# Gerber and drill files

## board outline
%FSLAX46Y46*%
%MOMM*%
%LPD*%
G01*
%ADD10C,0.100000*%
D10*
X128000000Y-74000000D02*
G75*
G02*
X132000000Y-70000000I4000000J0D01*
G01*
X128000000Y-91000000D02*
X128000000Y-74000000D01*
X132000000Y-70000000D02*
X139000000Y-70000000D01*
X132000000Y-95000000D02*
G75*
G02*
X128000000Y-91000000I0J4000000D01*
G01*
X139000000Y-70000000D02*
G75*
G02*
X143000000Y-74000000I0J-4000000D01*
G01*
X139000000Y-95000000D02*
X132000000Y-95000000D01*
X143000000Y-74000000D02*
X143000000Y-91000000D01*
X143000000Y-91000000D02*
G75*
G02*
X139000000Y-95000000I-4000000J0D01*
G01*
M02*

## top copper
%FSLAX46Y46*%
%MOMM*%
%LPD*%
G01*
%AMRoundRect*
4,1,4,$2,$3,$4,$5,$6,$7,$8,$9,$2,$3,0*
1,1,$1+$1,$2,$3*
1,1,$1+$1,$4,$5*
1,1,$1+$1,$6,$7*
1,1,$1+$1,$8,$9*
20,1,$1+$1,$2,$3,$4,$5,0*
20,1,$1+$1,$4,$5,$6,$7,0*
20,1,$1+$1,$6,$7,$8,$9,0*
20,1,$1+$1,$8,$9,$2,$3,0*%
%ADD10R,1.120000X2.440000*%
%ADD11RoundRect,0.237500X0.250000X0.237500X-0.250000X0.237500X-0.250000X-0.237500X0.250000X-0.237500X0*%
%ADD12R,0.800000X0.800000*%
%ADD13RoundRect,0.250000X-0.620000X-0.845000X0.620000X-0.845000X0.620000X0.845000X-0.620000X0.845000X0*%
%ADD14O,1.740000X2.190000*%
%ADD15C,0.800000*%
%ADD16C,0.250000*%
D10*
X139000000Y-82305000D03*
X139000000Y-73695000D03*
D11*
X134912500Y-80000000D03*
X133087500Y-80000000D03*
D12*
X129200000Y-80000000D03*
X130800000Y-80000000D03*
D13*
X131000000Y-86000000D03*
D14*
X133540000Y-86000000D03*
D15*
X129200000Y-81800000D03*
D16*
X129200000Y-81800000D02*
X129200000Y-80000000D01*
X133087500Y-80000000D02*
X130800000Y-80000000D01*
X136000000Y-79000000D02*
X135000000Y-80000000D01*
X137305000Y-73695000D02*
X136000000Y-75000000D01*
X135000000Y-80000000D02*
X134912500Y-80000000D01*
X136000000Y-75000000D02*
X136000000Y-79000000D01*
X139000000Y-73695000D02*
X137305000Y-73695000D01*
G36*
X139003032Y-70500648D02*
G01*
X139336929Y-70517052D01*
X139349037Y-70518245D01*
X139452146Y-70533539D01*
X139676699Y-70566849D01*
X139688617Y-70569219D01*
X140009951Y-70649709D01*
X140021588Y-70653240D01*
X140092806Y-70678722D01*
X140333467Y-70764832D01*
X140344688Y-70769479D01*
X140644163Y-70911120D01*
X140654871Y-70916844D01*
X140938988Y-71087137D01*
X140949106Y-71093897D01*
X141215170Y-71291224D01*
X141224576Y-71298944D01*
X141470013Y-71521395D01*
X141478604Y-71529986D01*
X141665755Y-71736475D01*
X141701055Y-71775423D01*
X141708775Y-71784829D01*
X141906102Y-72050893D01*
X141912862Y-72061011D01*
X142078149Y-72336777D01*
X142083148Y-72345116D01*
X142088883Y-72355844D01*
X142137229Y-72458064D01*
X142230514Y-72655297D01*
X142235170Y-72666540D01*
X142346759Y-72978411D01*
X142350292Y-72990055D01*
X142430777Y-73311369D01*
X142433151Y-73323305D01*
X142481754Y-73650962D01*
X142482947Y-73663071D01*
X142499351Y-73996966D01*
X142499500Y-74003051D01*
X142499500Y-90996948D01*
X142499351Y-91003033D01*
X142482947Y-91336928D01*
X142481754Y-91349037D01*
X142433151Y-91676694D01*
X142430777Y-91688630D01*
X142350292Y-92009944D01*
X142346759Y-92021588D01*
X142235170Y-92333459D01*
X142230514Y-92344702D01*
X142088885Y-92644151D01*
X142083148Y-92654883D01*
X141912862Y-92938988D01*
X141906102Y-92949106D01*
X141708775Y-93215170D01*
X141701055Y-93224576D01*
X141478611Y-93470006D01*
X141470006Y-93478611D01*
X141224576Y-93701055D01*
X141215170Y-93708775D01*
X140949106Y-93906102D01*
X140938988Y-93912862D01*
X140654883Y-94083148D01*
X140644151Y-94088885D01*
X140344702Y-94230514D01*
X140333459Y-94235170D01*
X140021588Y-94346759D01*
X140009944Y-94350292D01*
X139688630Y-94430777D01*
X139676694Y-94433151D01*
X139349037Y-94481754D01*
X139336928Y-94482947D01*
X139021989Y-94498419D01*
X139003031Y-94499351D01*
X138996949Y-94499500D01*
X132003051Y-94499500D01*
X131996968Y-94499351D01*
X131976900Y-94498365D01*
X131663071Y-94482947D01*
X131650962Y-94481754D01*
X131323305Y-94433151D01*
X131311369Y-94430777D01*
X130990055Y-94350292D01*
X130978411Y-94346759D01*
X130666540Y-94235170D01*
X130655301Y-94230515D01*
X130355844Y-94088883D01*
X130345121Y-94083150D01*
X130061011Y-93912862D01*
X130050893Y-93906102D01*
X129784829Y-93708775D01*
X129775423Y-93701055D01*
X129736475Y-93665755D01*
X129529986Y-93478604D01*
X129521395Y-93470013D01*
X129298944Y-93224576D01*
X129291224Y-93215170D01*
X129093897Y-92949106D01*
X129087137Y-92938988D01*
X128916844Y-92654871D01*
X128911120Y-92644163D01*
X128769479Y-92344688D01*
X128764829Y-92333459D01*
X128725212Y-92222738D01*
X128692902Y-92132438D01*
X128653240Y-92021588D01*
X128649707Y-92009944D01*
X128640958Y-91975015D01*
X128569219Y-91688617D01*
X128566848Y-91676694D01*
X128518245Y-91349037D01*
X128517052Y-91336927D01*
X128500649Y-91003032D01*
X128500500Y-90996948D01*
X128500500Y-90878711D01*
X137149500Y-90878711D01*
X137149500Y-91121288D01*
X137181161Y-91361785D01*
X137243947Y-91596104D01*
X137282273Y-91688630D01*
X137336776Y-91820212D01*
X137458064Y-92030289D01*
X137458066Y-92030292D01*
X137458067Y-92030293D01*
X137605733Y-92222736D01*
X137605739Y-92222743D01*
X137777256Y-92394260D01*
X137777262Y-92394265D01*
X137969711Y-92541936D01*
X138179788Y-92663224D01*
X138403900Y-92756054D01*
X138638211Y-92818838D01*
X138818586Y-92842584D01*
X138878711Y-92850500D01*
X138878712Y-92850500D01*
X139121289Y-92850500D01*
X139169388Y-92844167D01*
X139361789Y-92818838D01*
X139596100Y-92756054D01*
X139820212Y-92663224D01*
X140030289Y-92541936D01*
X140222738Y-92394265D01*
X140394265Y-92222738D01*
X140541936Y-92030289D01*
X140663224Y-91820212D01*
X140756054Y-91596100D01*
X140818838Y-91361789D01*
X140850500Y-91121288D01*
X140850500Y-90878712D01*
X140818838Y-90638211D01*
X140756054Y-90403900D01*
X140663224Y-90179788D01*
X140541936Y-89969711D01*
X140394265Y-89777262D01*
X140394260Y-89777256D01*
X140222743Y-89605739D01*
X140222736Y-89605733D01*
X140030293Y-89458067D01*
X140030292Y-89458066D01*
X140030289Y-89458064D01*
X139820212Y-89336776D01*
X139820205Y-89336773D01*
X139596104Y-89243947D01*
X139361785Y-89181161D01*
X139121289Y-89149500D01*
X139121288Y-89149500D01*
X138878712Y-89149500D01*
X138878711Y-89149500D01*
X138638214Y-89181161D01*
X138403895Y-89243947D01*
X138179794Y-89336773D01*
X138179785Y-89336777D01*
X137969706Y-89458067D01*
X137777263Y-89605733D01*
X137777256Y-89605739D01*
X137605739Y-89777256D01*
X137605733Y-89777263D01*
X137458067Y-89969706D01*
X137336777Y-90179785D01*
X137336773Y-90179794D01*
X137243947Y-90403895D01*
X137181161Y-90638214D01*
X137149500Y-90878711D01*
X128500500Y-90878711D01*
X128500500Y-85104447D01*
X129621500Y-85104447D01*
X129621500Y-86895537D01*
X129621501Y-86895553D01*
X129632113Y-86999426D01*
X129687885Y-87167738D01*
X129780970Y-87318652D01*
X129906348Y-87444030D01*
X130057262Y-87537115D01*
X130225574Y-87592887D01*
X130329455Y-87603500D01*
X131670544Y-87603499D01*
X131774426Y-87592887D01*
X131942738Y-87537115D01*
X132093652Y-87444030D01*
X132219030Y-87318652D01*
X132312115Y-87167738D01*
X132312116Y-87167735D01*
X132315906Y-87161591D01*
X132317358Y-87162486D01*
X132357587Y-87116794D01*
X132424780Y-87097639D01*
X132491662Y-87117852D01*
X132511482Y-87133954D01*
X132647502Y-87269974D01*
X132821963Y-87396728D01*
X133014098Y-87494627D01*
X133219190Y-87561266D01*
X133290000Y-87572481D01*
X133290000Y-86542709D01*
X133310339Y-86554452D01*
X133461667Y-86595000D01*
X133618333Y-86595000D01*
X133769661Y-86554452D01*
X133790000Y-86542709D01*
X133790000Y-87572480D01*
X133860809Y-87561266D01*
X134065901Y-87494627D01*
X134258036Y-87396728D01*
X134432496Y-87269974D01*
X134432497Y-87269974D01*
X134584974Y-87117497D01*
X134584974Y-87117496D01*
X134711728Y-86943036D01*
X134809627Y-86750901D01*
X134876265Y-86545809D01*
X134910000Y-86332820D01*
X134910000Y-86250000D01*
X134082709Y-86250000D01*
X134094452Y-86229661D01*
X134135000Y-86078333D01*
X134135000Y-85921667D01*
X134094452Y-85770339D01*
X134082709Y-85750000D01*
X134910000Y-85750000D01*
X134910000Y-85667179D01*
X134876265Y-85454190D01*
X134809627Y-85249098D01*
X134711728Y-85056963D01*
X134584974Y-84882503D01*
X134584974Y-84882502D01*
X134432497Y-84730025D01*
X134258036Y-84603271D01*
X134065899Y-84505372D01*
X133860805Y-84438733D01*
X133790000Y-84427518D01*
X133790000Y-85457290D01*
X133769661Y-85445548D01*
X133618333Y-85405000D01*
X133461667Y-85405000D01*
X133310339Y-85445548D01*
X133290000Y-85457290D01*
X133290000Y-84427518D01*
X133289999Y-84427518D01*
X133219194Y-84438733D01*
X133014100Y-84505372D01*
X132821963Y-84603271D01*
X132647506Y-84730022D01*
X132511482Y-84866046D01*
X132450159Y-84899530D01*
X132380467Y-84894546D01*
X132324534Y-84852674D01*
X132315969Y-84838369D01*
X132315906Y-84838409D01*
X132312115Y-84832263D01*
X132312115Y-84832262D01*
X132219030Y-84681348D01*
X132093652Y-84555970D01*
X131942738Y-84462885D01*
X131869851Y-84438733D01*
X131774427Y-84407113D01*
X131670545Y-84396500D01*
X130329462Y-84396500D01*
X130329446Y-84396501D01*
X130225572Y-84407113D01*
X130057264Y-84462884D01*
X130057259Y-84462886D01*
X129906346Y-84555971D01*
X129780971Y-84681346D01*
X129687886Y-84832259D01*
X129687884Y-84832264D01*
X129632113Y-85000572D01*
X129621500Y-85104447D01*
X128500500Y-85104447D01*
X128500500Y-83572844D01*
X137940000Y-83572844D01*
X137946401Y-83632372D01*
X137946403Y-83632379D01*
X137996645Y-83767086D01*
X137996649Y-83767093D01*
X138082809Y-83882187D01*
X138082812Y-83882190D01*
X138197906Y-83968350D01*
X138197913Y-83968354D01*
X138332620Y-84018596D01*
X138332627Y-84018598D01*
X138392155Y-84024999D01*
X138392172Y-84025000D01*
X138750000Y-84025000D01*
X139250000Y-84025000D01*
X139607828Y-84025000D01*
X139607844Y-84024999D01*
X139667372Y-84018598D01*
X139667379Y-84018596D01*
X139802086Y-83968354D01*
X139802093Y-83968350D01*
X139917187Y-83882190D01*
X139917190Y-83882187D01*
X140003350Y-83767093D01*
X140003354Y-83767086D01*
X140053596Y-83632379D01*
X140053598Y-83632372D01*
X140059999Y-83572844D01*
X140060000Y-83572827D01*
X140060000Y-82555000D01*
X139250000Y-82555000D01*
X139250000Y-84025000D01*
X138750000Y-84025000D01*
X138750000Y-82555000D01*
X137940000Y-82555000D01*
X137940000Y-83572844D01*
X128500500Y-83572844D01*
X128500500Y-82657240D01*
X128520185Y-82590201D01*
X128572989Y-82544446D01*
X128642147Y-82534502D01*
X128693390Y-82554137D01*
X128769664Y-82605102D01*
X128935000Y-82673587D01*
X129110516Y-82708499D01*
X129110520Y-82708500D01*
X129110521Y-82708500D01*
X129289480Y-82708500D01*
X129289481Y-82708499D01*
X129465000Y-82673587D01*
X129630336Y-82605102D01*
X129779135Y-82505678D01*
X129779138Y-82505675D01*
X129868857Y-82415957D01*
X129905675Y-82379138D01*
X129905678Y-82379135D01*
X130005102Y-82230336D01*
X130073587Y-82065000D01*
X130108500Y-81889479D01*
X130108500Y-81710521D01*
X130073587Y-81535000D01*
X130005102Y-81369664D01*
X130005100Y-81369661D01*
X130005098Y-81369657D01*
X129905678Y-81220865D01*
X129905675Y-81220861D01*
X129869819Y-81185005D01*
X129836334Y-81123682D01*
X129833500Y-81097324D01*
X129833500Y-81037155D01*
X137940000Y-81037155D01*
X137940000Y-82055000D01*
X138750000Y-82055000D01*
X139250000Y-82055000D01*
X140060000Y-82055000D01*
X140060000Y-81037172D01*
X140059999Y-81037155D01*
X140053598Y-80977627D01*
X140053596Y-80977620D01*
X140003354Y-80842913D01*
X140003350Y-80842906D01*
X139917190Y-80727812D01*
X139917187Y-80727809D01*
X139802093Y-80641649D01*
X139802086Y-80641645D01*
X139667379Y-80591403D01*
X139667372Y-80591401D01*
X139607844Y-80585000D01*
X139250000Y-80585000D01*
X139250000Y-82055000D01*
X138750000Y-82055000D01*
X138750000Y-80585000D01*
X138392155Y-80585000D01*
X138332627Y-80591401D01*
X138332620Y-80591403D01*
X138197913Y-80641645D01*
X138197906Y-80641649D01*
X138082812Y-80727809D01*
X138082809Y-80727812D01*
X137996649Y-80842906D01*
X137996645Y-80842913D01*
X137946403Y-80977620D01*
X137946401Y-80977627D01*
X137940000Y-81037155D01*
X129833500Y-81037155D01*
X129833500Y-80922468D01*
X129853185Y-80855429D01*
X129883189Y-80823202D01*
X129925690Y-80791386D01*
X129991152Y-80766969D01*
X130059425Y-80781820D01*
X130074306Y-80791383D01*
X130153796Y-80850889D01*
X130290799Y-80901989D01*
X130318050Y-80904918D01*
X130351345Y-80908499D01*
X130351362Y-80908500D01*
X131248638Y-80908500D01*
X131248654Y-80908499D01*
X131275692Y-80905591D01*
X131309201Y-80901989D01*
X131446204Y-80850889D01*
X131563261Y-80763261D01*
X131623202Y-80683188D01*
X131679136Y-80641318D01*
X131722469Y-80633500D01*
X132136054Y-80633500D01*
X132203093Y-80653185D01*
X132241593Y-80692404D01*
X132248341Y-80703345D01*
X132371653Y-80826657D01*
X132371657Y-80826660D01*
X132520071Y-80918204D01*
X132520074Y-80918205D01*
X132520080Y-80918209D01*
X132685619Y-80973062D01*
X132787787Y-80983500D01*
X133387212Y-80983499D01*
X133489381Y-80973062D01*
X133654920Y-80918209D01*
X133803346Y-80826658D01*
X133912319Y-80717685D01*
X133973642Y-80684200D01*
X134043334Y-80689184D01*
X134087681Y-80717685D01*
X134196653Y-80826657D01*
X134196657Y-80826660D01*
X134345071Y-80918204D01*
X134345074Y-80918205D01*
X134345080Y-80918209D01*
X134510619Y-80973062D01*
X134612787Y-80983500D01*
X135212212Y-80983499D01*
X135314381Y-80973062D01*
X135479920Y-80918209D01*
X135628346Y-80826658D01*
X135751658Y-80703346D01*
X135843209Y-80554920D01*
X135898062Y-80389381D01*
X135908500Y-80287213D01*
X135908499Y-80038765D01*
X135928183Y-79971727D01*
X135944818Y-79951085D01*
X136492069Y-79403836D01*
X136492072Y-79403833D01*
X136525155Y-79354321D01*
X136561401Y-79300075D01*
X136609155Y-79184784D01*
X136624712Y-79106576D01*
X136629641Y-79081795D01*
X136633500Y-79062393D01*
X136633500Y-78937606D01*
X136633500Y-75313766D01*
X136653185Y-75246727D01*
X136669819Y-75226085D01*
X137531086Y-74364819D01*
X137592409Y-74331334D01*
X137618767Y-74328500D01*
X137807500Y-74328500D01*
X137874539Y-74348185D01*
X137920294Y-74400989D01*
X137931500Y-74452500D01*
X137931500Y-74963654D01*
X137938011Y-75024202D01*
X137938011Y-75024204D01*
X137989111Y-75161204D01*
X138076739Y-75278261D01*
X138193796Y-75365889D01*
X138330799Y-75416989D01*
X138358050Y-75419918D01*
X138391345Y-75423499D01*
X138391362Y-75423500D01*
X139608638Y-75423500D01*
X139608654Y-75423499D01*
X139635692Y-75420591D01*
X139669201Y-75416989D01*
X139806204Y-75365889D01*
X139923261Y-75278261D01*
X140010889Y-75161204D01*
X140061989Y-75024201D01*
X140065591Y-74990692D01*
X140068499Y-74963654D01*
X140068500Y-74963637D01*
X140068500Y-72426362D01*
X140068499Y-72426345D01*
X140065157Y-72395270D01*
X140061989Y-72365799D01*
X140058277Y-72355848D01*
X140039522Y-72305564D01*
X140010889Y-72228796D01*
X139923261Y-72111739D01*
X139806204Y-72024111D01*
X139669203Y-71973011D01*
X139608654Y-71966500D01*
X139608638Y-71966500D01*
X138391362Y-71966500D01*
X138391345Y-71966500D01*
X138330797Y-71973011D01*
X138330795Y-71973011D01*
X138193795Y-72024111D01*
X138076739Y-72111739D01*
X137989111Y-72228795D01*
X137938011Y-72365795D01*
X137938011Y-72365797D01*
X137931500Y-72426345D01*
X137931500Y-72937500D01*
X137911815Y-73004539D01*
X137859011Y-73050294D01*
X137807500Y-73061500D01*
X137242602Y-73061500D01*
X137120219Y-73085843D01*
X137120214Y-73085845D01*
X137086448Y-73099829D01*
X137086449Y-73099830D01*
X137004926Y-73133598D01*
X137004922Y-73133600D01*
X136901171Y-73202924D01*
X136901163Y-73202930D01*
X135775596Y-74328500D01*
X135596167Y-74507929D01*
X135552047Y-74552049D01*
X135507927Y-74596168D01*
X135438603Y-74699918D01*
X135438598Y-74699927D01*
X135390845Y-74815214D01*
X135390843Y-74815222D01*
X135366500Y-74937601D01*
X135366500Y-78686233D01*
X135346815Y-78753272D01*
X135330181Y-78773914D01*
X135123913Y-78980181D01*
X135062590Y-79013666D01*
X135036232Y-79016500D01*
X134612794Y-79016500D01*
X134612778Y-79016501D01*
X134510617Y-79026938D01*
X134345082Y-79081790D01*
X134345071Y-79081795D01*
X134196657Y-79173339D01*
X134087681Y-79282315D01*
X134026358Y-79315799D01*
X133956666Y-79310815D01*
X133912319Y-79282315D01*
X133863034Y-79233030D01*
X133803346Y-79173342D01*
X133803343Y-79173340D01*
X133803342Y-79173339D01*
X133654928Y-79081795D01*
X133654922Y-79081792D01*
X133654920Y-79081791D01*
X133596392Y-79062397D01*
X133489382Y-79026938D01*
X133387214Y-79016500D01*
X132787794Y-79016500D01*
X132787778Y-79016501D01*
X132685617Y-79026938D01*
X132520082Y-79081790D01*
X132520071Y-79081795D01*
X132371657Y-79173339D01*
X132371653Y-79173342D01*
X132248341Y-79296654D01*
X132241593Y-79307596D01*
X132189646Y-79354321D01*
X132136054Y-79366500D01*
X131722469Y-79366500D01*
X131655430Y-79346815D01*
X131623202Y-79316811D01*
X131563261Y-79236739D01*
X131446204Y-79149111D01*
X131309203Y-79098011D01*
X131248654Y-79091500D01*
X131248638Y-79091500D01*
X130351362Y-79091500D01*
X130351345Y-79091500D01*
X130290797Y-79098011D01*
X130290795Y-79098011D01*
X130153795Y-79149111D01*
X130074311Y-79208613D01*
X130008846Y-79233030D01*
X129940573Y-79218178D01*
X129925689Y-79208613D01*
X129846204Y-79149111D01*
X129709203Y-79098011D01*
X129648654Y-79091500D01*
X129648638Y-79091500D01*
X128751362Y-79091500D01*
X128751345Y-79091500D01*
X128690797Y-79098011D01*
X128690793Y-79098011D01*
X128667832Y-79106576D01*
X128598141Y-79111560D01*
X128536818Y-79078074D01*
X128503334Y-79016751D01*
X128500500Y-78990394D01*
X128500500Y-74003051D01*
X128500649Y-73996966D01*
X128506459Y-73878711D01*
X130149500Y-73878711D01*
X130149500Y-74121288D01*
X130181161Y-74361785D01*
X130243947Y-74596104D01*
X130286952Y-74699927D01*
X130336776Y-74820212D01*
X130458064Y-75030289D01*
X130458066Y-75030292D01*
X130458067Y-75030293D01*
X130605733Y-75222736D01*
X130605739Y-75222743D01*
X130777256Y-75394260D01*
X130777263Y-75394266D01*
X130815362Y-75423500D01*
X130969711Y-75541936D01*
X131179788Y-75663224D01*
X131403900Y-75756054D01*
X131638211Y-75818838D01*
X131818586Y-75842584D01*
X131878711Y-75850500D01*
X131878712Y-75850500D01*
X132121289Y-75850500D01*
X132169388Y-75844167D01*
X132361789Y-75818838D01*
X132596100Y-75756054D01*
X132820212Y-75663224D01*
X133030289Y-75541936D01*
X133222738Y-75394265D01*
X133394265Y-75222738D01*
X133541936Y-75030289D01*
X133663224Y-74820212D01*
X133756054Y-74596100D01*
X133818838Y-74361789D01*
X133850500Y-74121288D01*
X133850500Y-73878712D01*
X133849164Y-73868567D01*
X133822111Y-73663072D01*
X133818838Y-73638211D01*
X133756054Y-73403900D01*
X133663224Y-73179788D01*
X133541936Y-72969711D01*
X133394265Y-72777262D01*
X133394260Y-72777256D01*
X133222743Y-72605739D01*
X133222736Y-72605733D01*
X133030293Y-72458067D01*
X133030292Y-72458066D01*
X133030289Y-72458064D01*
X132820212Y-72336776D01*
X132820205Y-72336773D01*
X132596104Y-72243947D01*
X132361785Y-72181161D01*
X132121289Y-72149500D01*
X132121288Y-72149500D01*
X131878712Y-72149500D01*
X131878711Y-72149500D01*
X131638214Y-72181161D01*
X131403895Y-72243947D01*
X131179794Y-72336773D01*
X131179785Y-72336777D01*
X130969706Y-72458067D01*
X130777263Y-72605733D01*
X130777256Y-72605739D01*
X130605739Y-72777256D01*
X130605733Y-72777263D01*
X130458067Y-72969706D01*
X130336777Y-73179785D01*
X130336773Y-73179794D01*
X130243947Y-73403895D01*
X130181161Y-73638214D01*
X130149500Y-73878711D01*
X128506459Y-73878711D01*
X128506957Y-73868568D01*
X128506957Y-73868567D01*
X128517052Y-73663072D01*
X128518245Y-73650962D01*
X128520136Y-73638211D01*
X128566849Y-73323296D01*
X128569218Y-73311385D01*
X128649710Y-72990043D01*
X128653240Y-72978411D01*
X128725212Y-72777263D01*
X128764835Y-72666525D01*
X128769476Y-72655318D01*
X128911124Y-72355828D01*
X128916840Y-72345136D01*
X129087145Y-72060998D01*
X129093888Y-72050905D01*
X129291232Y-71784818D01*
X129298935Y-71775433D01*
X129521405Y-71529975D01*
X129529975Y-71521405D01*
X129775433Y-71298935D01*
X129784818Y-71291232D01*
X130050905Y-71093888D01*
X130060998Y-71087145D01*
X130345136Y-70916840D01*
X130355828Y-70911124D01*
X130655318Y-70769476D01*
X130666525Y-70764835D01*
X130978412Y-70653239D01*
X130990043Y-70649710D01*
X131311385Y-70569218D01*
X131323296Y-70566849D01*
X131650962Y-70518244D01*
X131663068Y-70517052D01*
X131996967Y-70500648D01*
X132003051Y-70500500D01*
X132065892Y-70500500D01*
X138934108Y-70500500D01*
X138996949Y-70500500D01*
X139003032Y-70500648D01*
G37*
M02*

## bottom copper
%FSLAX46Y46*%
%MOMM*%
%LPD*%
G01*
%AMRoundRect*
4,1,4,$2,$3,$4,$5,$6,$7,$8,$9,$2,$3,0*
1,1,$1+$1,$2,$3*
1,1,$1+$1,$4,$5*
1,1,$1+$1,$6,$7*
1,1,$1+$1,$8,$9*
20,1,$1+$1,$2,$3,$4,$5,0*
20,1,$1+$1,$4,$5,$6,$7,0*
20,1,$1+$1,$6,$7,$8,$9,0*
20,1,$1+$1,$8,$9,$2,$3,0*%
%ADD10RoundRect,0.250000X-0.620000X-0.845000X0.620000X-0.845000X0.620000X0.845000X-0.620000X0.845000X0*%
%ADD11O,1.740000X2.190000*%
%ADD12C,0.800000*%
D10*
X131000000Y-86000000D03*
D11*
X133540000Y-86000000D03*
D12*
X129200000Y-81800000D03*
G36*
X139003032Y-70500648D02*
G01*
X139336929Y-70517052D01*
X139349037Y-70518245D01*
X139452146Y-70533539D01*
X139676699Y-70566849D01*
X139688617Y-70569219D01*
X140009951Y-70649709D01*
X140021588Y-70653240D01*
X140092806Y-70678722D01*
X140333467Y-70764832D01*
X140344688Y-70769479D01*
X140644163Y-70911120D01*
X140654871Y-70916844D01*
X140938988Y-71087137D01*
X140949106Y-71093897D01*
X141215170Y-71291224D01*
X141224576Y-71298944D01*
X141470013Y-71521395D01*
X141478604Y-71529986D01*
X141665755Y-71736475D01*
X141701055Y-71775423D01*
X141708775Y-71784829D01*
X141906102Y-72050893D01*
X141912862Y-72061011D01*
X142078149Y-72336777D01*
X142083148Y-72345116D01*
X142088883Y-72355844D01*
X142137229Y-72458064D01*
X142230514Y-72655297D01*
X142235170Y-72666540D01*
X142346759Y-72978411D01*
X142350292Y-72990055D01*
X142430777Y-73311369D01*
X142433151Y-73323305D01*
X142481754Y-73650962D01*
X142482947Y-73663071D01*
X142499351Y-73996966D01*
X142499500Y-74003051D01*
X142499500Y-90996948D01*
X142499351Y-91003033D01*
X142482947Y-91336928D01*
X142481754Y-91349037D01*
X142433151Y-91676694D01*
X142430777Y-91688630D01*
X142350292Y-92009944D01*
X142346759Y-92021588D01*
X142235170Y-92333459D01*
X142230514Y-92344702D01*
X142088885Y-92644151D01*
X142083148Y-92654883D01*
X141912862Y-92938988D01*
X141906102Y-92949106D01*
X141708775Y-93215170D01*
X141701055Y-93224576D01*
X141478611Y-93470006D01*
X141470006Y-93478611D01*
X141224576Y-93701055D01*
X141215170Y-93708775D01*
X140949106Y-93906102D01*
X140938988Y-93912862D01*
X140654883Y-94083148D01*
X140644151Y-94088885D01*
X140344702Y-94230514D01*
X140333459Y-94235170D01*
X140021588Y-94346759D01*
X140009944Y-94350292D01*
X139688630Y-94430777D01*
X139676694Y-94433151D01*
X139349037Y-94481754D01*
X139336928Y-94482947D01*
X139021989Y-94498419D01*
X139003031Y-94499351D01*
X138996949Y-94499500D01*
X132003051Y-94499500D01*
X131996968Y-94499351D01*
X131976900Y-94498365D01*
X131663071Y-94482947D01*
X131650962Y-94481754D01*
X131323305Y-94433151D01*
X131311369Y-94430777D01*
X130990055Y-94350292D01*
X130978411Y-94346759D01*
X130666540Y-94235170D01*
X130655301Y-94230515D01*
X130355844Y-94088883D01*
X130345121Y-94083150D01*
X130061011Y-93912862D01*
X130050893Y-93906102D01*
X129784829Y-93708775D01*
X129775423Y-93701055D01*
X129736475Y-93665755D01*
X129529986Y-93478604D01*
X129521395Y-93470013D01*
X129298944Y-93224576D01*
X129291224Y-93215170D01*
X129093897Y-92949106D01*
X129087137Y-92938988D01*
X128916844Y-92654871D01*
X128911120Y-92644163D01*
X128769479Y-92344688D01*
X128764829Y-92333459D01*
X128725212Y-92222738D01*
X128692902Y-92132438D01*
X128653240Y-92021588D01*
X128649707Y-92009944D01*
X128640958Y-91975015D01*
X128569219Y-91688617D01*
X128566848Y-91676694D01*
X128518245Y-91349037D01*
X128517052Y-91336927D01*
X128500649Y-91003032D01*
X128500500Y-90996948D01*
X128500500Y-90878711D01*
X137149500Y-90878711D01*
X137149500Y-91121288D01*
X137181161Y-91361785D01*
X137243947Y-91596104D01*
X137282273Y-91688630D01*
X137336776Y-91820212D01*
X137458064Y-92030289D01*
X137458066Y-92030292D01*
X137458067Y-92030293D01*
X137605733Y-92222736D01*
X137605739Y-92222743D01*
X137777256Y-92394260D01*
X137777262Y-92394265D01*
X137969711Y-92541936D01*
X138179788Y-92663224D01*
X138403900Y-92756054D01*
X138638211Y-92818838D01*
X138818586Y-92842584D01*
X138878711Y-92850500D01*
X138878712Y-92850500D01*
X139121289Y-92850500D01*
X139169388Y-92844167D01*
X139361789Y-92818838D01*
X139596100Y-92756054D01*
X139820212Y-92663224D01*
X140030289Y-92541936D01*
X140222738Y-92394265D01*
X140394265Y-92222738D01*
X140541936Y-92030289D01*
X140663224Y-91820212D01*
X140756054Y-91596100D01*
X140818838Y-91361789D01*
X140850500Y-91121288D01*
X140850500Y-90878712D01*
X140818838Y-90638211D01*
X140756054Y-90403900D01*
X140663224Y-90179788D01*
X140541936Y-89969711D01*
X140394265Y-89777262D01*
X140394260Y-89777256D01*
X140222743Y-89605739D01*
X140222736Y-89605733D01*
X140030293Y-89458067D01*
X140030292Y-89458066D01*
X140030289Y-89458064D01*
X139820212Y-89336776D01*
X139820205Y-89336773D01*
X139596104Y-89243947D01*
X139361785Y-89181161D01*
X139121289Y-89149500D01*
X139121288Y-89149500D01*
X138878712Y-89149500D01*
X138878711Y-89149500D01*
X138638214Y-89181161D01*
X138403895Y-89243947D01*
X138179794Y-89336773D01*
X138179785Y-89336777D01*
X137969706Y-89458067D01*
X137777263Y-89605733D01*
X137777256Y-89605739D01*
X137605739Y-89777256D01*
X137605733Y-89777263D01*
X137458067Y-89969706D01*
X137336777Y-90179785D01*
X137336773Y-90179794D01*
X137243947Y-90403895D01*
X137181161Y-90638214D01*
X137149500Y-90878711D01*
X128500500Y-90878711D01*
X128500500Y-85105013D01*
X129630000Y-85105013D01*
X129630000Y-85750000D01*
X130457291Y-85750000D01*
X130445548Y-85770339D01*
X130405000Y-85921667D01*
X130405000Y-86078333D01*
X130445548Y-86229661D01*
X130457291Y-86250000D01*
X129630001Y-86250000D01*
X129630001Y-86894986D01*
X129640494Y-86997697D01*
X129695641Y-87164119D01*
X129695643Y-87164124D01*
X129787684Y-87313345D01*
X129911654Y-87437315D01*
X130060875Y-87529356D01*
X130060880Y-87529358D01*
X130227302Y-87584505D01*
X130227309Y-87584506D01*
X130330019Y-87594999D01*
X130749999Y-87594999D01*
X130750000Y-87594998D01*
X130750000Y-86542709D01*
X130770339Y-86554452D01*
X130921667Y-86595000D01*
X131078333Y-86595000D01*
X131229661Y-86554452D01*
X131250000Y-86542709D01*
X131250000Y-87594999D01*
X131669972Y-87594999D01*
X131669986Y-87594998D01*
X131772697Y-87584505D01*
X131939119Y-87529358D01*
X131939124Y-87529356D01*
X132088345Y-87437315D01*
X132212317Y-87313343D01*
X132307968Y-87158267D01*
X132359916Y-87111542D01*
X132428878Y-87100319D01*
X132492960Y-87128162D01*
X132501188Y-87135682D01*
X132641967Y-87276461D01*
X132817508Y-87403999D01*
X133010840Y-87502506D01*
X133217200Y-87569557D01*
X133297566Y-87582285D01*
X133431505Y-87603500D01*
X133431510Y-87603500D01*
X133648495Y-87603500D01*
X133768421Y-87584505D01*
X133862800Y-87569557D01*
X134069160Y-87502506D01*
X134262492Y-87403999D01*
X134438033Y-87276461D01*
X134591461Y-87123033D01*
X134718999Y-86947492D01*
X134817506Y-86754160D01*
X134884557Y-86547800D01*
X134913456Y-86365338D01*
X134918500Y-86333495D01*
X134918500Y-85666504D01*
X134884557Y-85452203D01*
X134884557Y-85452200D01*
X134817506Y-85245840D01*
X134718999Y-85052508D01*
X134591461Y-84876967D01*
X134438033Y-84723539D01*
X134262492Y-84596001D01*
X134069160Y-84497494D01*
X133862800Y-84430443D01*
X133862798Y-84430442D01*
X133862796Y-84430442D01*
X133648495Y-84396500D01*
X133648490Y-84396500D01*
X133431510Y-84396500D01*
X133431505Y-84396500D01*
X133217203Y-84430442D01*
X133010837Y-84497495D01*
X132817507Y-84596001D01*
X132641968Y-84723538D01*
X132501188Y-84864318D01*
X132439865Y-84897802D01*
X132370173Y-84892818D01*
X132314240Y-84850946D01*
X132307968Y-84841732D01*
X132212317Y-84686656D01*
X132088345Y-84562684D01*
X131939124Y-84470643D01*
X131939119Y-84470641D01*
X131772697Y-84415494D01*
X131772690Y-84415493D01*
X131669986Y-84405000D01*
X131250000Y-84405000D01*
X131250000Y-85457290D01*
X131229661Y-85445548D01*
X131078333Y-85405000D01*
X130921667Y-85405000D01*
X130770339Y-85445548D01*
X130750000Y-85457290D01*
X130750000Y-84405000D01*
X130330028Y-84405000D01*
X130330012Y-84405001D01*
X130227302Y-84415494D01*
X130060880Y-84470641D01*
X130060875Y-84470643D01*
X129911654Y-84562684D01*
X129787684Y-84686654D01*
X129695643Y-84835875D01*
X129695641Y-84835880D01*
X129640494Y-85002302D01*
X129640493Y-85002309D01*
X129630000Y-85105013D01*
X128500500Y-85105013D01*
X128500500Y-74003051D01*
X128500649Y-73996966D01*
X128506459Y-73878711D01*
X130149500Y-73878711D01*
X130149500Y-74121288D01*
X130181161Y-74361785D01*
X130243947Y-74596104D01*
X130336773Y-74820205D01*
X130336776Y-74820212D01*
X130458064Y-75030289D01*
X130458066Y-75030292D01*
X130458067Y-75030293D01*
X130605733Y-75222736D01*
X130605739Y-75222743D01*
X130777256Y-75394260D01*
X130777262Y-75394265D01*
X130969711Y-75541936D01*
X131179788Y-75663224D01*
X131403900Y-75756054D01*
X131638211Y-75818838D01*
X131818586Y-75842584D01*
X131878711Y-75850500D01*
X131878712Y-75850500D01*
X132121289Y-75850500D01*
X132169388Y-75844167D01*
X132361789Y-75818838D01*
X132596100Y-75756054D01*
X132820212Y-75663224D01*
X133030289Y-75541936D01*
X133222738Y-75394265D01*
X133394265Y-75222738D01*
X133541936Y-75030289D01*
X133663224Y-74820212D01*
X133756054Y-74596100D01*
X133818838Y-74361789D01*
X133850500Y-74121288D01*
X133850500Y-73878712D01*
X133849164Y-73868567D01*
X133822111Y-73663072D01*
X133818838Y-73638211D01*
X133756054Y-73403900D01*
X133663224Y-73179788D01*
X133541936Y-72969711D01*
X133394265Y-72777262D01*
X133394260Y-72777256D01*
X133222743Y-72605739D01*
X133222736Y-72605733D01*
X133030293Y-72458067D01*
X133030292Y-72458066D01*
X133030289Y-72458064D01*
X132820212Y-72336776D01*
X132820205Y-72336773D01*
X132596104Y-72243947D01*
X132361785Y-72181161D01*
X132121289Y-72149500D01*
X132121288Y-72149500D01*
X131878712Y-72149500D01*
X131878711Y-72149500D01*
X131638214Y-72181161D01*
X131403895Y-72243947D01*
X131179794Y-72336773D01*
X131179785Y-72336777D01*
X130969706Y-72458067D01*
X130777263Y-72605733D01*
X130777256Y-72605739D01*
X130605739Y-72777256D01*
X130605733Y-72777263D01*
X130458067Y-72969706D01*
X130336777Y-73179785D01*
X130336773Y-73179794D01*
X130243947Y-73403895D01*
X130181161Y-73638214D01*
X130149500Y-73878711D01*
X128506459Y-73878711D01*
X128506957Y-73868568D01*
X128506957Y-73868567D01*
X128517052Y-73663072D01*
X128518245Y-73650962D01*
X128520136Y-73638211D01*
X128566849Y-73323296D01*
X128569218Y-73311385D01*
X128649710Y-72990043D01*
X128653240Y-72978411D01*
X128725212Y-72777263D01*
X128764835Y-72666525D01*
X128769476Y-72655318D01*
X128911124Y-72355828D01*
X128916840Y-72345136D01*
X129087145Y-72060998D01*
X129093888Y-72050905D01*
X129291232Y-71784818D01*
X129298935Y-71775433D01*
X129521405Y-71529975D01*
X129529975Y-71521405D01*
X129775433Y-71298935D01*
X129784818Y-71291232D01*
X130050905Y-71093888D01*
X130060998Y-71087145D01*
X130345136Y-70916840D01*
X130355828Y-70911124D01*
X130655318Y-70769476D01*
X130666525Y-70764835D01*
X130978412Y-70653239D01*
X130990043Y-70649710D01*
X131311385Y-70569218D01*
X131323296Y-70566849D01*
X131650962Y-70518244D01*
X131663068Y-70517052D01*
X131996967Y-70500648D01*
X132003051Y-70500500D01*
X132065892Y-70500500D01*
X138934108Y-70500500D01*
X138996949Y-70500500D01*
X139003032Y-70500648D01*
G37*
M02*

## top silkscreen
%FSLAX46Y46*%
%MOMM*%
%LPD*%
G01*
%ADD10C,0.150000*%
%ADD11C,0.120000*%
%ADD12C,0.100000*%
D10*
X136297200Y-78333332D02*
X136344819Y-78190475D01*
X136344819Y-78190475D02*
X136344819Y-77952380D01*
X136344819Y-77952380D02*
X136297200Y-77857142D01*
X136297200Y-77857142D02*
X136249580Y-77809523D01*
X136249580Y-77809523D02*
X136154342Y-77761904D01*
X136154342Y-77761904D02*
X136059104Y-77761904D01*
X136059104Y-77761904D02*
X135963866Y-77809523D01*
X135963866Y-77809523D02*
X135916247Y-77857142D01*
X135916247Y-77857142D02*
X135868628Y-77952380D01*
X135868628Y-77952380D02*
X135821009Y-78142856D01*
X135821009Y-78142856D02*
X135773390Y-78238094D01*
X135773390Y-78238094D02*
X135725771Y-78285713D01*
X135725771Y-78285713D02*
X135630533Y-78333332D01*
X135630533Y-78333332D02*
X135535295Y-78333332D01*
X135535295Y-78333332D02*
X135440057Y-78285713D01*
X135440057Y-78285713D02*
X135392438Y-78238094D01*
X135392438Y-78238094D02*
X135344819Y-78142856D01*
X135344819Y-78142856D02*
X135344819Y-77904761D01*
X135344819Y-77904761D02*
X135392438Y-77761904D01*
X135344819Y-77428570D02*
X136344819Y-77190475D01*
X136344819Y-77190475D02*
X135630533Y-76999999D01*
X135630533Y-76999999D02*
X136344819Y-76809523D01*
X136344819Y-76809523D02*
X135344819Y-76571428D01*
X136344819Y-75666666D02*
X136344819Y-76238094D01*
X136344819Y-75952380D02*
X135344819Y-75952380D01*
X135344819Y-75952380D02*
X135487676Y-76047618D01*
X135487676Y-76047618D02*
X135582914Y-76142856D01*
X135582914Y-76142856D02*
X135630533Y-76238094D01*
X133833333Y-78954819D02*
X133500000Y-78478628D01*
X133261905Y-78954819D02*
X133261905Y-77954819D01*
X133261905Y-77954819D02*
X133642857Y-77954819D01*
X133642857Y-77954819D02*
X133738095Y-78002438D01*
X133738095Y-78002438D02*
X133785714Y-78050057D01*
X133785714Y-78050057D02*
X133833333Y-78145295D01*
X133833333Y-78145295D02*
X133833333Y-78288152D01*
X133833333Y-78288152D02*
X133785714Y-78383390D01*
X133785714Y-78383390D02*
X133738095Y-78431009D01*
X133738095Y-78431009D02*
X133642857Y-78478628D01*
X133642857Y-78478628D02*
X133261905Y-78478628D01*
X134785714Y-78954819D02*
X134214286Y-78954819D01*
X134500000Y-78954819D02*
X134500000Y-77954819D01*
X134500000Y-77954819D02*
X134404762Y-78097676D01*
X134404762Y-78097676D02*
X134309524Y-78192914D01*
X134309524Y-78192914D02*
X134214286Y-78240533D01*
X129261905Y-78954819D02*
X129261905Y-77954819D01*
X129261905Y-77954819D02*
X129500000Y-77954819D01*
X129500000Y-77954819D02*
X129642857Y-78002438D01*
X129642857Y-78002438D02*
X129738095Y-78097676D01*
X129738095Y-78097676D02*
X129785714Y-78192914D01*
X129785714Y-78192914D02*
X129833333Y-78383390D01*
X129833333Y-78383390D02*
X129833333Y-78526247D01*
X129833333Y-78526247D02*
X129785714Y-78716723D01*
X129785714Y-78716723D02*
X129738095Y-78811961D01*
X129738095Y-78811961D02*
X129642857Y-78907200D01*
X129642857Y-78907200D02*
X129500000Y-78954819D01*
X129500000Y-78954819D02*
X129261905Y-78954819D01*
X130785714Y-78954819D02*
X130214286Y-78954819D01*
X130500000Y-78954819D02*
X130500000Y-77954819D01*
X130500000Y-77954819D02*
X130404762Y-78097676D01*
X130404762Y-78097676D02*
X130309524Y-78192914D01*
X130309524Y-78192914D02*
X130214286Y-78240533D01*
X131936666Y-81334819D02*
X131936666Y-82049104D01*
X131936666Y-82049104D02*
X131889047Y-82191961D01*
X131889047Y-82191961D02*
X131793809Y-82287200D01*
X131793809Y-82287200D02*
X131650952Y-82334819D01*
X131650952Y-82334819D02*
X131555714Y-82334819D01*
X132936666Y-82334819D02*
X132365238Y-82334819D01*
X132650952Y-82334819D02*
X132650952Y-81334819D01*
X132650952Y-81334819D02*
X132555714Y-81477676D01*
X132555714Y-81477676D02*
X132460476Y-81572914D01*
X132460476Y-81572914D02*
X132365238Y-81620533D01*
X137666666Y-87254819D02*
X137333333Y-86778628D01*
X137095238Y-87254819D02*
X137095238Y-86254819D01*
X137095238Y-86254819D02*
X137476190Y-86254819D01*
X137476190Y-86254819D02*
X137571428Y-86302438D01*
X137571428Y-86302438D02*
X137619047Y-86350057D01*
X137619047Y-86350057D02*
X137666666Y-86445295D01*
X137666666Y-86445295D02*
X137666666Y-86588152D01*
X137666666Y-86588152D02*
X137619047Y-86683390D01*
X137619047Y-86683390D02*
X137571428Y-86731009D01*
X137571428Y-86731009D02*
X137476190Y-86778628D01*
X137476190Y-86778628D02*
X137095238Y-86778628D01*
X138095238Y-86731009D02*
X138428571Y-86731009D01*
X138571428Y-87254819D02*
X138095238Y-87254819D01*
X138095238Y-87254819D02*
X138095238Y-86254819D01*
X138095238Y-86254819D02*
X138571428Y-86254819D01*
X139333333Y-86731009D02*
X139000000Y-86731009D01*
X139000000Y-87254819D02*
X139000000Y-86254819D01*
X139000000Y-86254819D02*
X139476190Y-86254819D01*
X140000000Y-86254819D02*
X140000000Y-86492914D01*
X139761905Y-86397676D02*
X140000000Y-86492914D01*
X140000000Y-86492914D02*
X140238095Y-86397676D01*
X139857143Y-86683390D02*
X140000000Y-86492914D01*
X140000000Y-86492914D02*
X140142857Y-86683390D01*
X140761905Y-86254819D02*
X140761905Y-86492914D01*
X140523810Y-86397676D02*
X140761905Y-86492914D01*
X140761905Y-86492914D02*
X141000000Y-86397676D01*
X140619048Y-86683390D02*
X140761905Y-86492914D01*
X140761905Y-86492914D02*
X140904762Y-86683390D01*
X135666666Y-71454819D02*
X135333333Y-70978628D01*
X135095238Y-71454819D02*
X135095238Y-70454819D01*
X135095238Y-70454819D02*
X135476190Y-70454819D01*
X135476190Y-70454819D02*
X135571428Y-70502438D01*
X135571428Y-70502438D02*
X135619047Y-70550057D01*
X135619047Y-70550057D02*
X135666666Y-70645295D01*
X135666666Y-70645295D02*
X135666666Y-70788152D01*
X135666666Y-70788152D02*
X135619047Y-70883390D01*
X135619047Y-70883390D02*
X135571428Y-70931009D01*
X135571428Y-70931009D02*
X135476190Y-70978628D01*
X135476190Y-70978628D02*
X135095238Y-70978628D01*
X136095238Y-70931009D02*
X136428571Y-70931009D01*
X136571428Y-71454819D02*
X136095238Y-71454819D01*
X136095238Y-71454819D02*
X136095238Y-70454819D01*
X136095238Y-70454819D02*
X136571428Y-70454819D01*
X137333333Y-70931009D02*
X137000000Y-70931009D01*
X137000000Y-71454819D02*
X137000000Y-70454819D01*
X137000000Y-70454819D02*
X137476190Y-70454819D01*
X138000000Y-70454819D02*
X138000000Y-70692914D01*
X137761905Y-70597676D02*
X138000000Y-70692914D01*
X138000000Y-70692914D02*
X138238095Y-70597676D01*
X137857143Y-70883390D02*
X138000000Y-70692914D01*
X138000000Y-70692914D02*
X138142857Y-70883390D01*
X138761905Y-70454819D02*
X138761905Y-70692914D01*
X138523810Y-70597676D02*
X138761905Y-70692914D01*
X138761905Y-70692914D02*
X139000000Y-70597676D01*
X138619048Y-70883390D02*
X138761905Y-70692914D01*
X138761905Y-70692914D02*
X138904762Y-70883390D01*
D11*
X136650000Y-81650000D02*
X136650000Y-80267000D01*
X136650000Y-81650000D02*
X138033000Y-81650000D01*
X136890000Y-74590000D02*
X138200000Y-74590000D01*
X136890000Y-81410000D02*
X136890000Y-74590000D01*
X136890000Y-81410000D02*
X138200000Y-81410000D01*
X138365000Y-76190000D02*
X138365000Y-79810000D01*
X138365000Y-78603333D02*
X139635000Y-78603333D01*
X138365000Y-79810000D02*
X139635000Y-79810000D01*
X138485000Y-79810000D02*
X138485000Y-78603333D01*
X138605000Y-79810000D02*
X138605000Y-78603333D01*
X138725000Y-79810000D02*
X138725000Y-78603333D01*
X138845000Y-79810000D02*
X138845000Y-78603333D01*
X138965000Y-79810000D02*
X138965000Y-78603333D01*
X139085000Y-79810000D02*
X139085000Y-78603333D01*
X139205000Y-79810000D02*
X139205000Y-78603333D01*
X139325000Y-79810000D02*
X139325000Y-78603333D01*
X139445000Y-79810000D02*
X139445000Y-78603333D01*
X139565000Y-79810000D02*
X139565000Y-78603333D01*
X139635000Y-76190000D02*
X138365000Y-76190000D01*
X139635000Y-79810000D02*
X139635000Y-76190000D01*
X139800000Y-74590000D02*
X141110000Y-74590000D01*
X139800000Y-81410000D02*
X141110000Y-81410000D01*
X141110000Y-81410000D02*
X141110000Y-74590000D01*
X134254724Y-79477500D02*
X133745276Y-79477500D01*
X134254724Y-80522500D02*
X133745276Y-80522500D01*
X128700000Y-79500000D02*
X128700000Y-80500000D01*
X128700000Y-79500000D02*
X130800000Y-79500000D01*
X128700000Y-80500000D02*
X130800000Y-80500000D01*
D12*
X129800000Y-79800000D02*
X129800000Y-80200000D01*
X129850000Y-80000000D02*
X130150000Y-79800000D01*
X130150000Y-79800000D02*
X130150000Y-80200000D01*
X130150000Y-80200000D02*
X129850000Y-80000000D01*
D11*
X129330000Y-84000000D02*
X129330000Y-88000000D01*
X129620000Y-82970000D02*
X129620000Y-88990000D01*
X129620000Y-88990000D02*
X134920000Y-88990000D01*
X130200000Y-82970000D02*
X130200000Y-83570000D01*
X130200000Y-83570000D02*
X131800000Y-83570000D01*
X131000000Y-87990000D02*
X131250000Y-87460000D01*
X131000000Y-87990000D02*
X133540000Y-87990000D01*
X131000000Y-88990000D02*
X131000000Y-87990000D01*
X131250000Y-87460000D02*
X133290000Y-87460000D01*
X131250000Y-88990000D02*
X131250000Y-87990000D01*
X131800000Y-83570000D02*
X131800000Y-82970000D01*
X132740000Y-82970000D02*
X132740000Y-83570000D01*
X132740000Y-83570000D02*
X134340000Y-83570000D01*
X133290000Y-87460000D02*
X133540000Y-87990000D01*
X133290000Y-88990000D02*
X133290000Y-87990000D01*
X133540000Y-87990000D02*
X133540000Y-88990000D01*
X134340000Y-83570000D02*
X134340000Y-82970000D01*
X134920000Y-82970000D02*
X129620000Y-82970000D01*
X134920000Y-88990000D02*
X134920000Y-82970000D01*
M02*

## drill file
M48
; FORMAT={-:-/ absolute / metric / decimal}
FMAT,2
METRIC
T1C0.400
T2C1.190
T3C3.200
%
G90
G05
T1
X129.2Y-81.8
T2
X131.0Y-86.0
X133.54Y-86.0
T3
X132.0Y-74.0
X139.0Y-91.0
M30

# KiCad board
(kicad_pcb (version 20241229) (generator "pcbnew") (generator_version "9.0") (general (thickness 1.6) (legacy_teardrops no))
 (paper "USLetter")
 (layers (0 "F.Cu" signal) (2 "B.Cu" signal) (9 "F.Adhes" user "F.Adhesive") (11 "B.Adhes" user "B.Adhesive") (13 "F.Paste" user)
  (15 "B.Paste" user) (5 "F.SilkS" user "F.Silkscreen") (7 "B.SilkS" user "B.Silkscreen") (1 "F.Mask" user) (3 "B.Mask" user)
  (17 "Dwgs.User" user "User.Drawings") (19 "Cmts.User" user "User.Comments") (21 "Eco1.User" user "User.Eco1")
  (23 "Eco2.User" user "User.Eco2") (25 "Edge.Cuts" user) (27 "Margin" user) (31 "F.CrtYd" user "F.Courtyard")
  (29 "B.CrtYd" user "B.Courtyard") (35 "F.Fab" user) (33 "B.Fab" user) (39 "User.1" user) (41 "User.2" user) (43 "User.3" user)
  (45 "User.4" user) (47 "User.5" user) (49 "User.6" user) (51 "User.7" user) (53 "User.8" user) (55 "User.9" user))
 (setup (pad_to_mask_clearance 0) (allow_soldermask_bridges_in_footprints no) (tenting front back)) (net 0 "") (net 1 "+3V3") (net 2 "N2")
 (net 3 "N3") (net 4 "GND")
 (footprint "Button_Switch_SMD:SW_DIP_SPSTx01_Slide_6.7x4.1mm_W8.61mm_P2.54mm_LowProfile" (layer "F.Cu") (at 139 78 90)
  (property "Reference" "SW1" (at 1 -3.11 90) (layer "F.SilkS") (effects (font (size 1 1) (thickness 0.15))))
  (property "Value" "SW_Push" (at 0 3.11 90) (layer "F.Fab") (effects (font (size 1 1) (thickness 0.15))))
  (fp_line (start -3.65 -2.35) (end -2.267 -2.35) (stroke (width 0.12) (type solid)) (layer "F.SilkS"))
  (fp_line (start -3.65 -2.35) (end -3.65 -0.967) (stroke (width 0.12) (type solid)) (layer "F.SilkS"))
  (fp_line (start 3.41 -2.11) (end 3.41 -0.8) (stroke (width 0.12) (type solid)) (layer "F.SilkS"))
  (fp_line (start -3.41 -2.11) (end 3.41 -2.11) (stroke (width 0.12) (type solid)) (layer "F.SilkS"))
  (fp_line (start -3.41 -2.11) (end -3.41 -0.8) (stroke (width 0.12) (type solid)) (layer "F.SilkS"))
  (fp_line (start 1.81 -0.635) (end -1.81 -0.635) (stroke (width 0.12) (type solid)) (layer "F.SilkS"))
  (fp_line (start -0.603333 -0.635) (end -0.603333 0.635) (stroke (width 0.12) (type solid)) (layer "F.SilkS"))
  (fp_line (start -1.81 -0.635) (end -1.81 0.635) (stroke (width 0.12) (type solid)) (layer "F.SilkS"))
  (fp_line (start -1.81 -0.515) (end -0.603333 -0.515) (stroke (width 0.12) (type solid)) (layer "F.SilkS"))
  (fp_line (start -1.81 -0.395) (end -0.603333 -0.395) (stroke (width 0.12) (type solid)) (layer "F.SilkS"))
  (fp_line (start -1.81 -0.275) (end -0.603333 -0.275) (stroke (width 0.12) (type solid)) (layer "F.SilkS"))
  (fp_line (start -1.81 -0.155) (end -0.603333 -0.155) (stroke (width 0.12) (type solid)) (layer "F.SilkS"))
  (fp_line (start -1.81 -0.035) (end -0.603333 -0.035) (stroke (width 0.12) (type solid)) (layer "F.SilkS"))
  (fp_line (start -1.81 0.085) (end -0.603333 0.085) (stroke (width 0.12) (type solid)) (layer "F.SilkS"))
  (fp_line (start -1.81 0.205) (end -0.603333 0.205) (stroke (width 0.12) (type solid)) (layer "F.SilkS"))
  (fp_line (start -1.81 0.325) (end -0.603333 0.325) (stroke (width 0.12) (type solid)) (layer "F.SilkS"))
  (fp_line (start -1.81 0.445) (end -0.603333 0.445) (stroke (width 0.12) (type solid)) (layer "F.SilkS"))
  (fp_line (start -1.81 0.565) (end -0.603333 0.565) (stroke (width 0.12) (type solid)) (layer "F.SilkS"))
  (fp_line (start 1.81 0.635) (end 1.81 -0.635) (stroke (width 0.12) (type solid)) (layer "F.SilkS"))
  (fp_line (start -1.81 0.635) (end 1.81 0.635) (stroke (width 0.12) (type solid)) (layer "F.SilkS"))
  (fp_line (start 3.41 0.8) (end 3.41 2.11) (stroke (width 0.12) (type solid)) (layer "F.SilkS"))
  (fp_line (start -3.41 0.8) (end -3.41 2.11) (stroke (width 0.12) (type solid)) (layer "F.SilkS"))
  (fp_line (start -3.41 2.11) (end 3.41 2.11) (stroke (width 0.12) (type solid)) (layer "F.SilkS"))
  (pad "1" smd rect (at -4.305 0 90) (size 2.44 1.12) (layers "F.Cu" "F.Mask" "F.Paste") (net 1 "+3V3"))
  (pad "2" smd rect (at 4.305 0 90) (size 2.44 1.12) (layers "F.Cu" "F.Mask" "F.Paste") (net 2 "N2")))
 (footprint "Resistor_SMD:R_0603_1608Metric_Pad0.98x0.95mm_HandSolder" (layer "F.Cu") (at 134 80 180)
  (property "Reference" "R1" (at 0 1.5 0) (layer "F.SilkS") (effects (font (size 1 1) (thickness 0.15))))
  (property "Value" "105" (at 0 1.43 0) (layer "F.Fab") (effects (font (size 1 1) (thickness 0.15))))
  (fp_line (start -0.254724 0.5225) (end 0.254724 0.5225) (stroke (width 0.12) (type solid)) (layer "F.SilkS"))
  (fp_line (start -0.254724 -0.5225) (end 0.254724 -0.5225) (stroke (width 0.12) (type solid)) (layer "F.SilkS"))
  (pad "1" smd roundrect (at -0.9125 0 180) (size 0.975 0.95) (layers "F.Cu" "F.Mask" "F.Paste") (roundrect_rratio 0.25) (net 2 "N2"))
  (pad "2" smd roundrect (at 0.9125 0 180) (size 0.975 0.95) (layers "F.Cu" "F.Mask" "F.Paste") (roundrect_rratio 0.25) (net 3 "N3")))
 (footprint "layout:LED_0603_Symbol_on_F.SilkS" (layer "F.Cu") (at 130 80)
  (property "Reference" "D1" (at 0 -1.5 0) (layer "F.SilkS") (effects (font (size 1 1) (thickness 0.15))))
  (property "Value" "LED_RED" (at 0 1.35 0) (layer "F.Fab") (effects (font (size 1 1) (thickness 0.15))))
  (fp_line (start -1.3 -0.5) (end -1.3 0.5) (stroke (width 0.12) (type solid)) (layer "F.SilkS"))
  (fp_line (start -1.3 -0.5) (end 0.8 -0.5) (stroke (width 0.12) (type solid)) (layer "F.SilkS"))
  (fp_line (start -1.3 0.5) (end 0.8 0.5) (stroke (width 0.12) (type solid)) (layer "F.SilkS"))
  (fp_line (start -0.2 -0.2) (end -0.2 0.2) (stroke (width 0.1) (type solid)) (layer "F.SilkS"))
  (fp_line (start -0.15 0) (end 0.15 -0.2) (stroke (width 0.1) (type solid)) (layer "F.SilkS"))
  (fp_line (start 0.15 -0.2) (end 0.15 0.2) (stroke (width 0.1) (type solid)) (layer "F.SilkS"))
  (fp_line (start 0.15 0.2) (end -0.15 0) (stroke (width 0.1) (type solid)) (layer "F.SilkS"))
  (pad "1" smd rect (at -0.8 0 180) (size 0.8 0.8) (layers "F.Cu" "F.Mask" "F.Paste") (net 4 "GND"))
  (pad "2" smd rect (at 0.8 0 180) (size 0.8 0.8) (layers "F.Cu" "F.Mask" "F.Paste") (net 3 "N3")))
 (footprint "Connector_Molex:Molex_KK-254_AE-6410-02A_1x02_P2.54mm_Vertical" (layer "F.Cu") (at 131 86)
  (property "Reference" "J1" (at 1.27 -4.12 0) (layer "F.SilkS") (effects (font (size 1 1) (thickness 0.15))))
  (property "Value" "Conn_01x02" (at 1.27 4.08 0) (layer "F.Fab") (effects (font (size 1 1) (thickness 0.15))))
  (fp_line (start -1.67 -2) (end -1.67 2) (stroke (width 0.12) (type solid)) (layer "F.SilkS"))
  (fp_line (start -1.38 -3.03) (end -1.38 2.99) (stroke (width 0.12) (type solid)) (layer "F.SilkS"))
  (fp_line (start -1.38 2.99) (end 3.92 2.99) (stroke (width 0.12) (type solid)) (layer "F.SilkS"))
  (fp_line (start -0.8 -3.03) (end -0.8 -2.43) (stroke (width 0.12) (type solid)) (layer "F.SilkS"))
  (fp_line (start -0.8 -2.43) (end 0.8 -2.43) (stroke (width 0.12) (type solid)) (layer "F.SilkS"))
  (fp_line (start 0 1.99) (end 0.25 1.46) (stroke (width 0.12) (type solid)) (layer "F.SilkS"))
  (fp_line (start 0 1.99) (end 2.54 1.99) (stroke (width 0.12) (type solid)) (layer "F.SilkS"))
  (fp_line (start 0 2.99) (end 0 1.99) (stroke (width 0.12) (type solid)) (layer "F.SilkS"))
  (fp_line (start 0.25 1.46) (end 2.29 1.46) (stroke (width 0.12) (type solid)) (layer "F.SilkS"))
  (fp_line (start 0.25 2.99) (end 0.25 1.99) (stroke (width 0.12) (type solid)) (layer "F.SilkS"))
  (fp_line (start 0.8 -2.43) (end 0.8 -3.03) (stroke (width 0.12) (type solid)) (layer "F.SilkS"))
  (fp_line (start 1.74 -3.03) (end 1.74 -2.43) (stroke (width 0.12) (type solid)) (layer "F.SilkS"))
  (fp_line (start 1.74 -2.43) (end 3.34 -2.43) (stroke (width 0.12) (type solid)) (layer "F.SilkS"))
  (fp_line (start 2.29 1.46) (end 2.54 1.99) (stroke (width 0.12) (type solid)) (layer "F.SilkS"))
  (fp_line (start 2.29 2.99) (end 2.29 1.99) (stroke (width 0.12) (type solid)) (layer "F.SilkS"))
  (fp_line (start 2.54 1.99) (end 2.54 2.99) (stroke (width 0.12) (type solid)) (layer "F.SilkS"))
  (fp_line (start 3.34 -2.43) (end 3.34 -3.03) (stroke (width 0.12) (type solid)) (layer "F.SilkS"))
  (fp_line (start 3.92 -3.03) (end -1.38 -3.03) (stroke (width 0.12) (type solid)) (layer "F.SilkS"))
  (fp_line (start 3.92 2.99) (end 3.92 -3.03) (stroke (width 0.12) (type solid)) (layer "F.SilkS"))
  (pad "1" thru_hole roundrect (at 0 0) (size 1.74 2.19) (drill 1.19) (layers "*.Cu" "*.Mask") (remove_unused_layers no)
   (roundrect_rratio 0.143678) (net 4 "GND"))
  (pad "2" thru_hole oval (at 2.54 0) (size 1.74 2.19) (drill 1.19) (layers "*.Cu" "*.Mask") (remove_unused_layers no) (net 1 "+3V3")))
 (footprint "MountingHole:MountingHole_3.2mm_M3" (layer "F.Cu") (at 139 91)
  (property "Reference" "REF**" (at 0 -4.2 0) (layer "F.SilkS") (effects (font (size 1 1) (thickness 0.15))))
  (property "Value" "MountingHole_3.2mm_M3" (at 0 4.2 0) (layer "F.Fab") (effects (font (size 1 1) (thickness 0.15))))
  (pad "" np_thru_hole circle (at 0 0) (size 3.2 3.2) (drill 3.2) (layers "*.Cu" "*.Mask")))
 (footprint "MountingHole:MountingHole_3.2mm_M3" (layer "F.Cu") (at 132 74)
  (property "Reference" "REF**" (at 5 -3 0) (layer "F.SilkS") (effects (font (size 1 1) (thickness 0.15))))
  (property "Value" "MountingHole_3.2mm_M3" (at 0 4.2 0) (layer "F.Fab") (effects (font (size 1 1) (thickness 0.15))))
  (pad "" np_thru_hole circle (at 0 0) (size 3.2 3.2) (drill 3.2) (layers "*.Cu" "*.Mask")))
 (gr_arc (start 128 74) (mid 129.171573 71.171573) (end 132 70) (stroke (width 0.1) (type default)) (layer "Edge.Cuts"))
 (gr_line (start 128 91) (end 128 74) (stroke (width 0.1) (type default)) (layer "Edge.Cuts"))
 (gr_line (start 132 70) (end 139 70) (stroke (width 0.1) (type default)) (layer "Edge.Cuts"))
 (gr_arc (start 132 95) (mid 129.171573 93.828427) (end 128 91) (stroke (width 0.1) (type default)) (layer "Edge.Cuts"))
 (gr_arc (start 139 70) (mid 141.828427 71.171573) (end 143 74) (stroke (width 0.1) (type default)) (layer "Edge.Cuts"))
 (gr_line (start 139 95) (end 132 95) (stroke (width 0.1) (type default)) (layer "Edge.Cuts"))
 (gr_line (start 143 74) (end 143 91) (stroke (width 0.1) (type default)) (layer "Edge.Cuts"))
 (gr_arc (start 143 91) (mid 141.828427 93.828427) (end 139 95) (stroke (width 0.1) (type default)) (layer "Edge.Cuts"))
 (segment (start 129.2 81.8) (end 129.2 80) (width 0.25) (layer "F.Cu") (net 4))
 (via (at 129.2 81.8) (size 0.8) (drill 0.4) (layers "F.Cu" "B.Cu") (free yes) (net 4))
 (segment (start 133.0875 80) (end 130.8 80) (width 0.25) (layer "F.Cu") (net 3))
 (segment (start 136 79) (end 135 80) (width 0.25) (layer "F.Cu") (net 2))
 (segment (start 137.305 73.695) (end 136 75) (width 0.25) (layer "F.Cu") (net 2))
 (segment (start 135 80) (end 134.9125 80) (width 0.25) (layer "F.Cu") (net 2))
 (segment (start 136 75) (end 136 79) (width 0.25) (layer "F.Cu") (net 2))
 (segment (start 139 73.695) (end 137.305 73.695) (width 0.25) (layer "F.Cu") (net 2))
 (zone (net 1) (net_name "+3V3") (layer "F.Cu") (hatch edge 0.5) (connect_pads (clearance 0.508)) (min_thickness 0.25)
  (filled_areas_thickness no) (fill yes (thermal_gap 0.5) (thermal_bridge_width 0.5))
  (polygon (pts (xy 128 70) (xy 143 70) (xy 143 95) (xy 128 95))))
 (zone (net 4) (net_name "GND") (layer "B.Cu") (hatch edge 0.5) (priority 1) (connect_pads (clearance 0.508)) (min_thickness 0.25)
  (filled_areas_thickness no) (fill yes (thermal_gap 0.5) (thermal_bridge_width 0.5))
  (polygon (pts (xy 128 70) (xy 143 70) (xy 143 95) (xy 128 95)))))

